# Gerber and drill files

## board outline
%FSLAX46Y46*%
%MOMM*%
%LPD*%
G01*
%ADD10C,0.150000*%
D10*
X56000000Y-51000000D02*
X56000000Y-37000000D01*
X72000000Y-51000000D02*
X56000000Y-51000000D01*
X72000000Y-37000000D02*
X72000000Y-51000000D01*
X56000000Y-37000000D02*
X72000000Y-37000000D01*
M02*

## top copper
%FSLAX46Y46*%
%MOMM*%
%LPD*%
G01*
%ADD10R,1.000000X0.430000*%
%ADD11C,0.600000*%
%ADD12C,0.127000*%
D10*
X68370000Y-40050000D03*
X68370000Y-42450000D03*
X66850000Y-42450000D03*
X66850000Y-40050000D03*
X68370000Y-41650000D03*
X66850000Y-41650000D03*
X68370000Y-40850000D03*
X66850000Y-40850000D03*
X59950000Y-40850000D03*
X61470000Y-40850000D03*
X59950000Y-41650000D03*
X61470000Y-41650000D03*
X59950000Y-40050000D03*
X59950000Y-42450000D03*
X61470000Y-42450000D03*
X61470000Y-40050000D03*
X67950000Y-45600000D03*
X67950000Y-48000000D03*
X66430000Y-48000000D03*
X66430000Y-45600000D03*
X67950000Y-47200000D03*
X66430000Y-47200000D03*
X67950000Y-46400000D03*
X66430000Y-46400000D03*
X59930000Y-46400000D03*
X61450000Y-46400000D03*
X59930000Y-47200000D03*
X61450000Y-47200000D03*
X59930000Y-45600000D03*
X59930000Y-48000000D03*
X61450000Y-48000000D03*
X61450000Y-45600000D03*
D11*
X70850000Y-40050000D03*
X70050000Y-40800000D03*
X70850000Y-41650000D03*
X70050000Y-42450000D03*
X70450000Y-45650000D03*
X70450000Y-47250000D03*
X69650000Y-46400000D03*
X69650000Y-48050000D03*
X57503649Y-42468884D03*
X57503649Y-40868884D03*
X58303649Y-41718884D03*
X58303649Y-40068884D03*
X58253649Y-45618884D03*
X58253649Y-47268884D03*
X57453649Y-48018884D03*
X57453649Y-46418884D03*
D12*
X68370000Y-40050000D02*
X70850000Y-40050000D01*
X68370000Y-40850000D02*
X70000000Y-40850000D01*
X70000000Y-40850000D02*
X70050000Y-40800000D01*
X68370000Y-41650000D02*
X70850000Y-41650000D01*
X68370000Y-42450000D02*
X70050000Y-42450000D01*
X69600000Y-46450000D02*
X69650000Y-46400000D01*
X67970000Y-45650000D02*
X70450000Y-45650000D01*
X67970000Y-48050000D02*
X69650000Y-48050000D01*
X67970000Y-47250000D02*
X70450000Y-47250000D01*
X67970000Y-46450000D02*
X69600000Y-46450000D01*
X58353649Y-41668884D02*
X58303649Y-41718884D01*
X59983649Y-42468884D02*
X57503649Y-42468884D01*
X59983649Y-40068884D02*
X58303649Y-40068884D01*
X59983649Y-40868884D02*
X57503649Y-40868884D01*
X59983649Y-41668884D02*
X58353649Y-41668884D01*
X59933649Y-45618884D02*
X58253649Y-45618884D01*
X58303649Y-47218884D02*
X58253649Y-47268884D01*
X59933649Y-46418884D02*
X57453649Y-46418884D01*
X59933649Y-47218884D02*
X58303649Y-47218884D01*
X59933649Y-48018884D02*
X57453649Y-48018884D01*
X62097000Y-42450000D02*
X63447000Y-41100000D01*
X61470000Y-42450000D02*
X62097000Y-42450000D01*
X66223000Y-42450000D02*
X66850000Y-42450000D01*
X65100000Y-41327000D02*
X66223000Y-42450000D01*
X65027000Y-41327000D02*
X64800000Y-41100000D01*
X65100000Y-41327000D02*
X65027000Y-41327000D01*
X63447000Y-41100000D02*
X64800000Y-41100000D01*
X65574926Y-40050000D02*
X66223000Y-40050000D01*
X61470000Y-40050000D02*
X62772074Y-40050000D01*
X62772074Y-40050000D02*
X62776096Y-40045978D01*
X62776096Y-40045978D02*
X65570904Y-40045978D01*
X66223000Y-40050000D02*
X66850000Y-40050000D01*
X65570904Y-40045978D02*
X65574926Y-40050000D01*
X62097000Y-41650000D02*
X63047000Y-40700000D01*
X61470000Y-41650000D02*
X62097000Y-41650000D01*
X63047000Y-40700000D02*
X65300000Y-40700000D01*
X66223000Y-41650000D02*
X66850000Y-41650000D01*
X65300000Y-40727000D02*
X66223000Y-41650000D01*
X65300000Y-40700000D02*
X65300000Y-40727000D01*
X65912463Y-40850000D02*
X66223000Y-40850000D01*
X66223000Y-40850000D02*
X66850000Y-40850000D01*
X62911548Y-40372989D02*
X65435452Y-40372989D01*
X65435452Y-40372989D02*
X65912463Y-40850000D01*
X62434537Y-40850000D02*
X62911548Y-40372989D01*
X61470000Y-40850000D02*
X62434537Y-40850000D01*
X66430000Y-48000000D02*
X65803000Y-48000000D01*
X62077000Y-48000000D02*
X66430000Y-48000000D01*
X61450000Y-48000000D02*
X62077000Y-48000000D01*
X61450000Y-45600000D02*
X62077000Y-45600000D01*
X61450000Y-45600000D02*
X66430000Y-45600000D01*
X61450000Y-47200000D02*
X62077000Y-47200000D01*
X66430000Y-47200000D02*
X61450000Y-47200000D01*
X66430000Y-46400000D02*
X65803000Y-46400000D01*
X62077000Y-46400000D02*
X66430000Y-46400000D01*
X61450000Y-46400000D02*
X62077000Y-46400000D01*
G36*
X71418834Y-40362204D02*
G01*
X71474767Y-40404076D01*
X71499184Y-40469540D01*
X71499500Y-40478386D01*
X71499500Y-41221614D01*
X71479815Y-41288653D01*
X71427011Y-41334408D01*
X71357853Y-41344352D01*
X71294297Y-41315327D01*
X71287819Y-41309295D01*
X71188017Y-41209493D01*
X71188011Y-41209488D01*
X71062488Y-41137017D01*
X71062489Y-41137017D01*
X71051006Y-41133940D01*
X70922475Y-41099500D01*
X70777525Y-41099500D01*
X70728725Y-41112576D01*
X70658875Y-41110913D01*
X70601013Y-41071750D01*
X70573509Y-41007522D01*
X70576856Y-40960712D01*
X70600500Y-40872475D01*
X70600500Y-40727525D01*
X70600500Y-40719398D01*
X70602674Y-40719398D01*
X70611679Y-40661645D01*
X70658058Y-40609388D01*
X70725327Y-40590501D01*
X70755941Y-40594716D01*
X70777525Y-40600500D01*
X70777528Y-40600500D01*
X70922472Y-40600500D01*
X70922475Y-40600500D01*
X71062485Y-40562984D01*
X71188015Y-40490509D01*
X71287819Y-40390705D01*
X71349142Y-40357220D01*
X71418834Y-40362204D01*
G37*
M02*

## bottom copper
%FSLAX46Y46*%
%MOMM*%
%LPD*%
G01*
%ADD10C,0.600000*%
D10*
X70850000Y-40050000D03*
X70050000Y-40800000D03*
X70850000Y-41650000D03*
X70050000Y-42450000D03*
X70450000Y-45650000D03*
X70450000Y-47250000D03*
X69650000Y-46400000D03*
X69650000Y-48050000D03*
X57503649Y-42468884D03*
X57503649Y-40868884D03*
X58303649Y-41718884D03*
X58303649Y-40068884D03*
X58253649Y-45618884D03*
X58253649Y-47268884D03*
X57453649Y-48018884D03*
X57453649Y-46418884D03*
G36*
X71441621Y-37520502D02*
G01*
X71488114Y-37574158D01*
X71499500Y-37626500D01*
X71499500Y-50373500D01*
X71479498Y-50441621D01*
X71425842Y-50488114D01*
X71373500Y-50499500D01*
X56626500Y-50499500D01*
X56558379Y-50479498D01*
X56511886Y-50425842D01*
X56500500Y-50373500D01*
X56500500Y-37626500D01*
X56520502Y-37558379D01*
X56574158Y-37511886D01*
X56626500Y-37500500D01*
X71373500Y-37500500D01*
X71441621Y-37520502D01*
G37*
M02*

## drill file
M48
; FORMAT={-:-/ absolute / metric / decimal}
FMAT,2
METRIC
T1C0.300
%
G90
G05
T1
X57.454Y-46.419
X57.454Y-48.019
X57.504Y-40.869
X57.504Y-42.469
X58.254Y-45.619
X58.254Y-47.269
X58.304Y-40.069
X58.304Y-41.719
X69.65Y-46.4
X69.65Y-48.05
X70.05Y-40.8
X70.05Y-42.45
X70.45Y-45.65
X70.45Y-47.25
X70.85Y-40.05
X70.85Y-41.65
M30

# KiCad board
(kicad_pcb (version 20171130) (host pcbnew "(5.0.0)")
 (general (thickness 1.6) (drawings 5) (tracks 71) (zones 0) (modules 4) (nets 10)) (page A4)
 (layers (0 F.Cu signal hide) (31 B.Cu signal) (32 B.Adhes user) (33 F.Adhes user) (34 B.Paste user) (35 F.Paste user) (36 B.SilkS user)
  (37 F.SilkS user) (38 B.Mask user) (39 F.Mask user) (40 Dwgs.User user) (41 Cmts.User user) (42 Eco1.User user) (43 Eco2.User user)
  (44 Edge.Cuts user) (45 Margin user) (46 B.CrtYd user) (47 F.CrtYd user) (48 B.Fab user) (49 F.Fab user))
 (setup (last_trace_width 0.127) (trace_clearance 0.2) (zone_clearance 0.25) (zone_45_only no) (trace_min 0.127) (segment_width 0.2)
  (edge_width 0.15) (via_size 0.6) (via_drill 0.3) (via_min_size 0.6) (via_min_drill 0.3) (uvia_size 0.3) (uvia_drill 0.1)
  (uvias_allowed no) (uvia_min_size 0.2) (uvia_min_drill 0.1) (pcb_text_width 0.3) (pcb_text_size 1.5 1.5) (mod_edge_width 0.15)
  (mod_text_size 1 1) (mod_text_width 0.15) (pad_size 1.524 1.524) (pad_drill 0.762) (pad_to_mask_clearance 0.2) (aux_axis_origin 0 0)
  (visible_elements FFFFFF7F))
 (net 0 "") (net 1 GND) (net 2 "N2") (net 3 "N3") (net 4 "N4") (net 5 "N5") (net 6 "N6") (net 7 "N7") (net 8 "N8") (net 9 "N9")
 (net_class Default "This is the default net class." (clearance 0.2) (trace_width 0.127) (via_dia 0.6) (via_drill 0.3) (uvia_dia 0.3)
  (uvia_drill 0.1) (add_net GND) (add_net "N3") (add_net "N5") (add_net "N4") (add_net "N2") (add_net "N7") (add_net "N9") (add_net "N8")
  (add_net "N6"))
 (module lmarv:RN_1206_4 (layer F.Cu) (at 67.61 41.25)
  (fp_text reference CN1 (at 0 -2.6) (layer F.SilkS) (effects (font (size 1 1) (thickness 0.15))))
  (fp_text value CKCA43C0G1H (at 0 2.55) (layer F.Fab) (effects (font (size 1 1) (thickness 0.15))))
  (pad 8 smd rect (at 0.76 -1.2 180) (size 1 0.43) (layers F.Cu F.Paste F.Mask) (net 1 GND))
  (pad 5 smd rect (at 0.76 1.2 180) (size 1 0.43) (layers F.Cu F.Paste F.Mask) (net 1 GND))
  (pad 4 smd rect (at -0.76 1.2 180) (size 1 0.43) (layers F.Cu F.Paste F.Mask) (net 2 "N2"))
  (pad 1 smd rect (at -0.76 -1.2 180) (size 1 0.43) (layers F.Cu F.Paste F.Mask) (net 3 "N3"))
  (pad 6 smd rect (at 0.76 0.4 180) (size 1 0.43) (layers F.Cu F.Paste F.Mask) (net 1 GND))
  (pad 3 smd rect (at -0.76 0.4 180) (size 1 0.43) (layers F.Cu F.Paste F.Mask) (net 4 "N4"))
  (pad 7 smd rect (at 0.76 -0.4 180) (size 1 0.43) (layers F.Cu F.Paste F.Mask) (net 1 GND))
  (pad 2 smd rect (at -0.76 -0.4 180) (size 1 0.43) (layers F.Cu F.Paste F.Mask) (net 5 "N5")))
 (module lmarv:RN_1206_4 (layer F.Cu) (at 60.71 41.25)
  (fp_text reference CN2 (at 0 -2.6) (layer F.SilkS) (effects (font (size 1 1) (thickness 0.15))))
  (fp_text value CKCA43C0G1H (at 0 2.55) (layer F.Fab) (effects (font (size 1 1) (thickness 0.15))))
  (pad 2 smd rect (at -0.76 -0.4 180) (size 1 0.43) (layers F.Cu F.Paste F.Mask) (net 1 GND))
  (pad 7 smd rect (at 0.76 -0.4 180) (size 1 0.43) (layers F.Cu F.Paste F.Mask) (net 5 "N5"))
  (pad 3 smd rect (at -0.76 0.4 180) (size 1 0.43) (layers F.Cu F.Paste F.Mask) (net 1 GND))
  (pad 6 smd rect (at 0.76 0.4 180) (size 1 0.43) (layers F.Cu F.Paste F.Mask) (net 4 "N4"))
  (pad 1 smd rect (at -0.76 -1.2 180) (size 1 0.43) (layers F.Cu F.Paste F.Mask) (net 1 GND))
  (pad 4 smd rect (at -0.76 1.2 180) (size 1 0.43) (layers F.Cu F.Paste F.Mask) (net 1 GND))
  (pad 5 smd rect (at 0.76 1.2 180) (size 1 0.43) (layers F.Cu F.Paste F.Mask) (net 2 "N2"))
  (pad 8 smd rect (at 0.76 -1.2 180) (size 1 0.43) (layers F.Cu F.Paste F.Mask) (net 3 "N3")))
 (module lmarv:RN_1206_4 (layer F.Cu) (at 67.19 46.8)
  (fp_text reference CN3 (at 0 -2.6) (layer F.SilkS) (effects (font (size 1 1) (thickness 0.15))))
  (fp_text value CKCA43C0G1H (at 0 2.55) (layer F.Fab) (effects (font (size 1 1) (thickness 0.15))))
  (pad 8 smd rect (at 0.76 -1.2 180) (size 1 0.43) (layers F.Cu F.Paste F.Mask) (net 1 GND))
  (pad 5 smd rect (at 0.76 1.2 180) (size 1 0.43) (layers F.Cu F.Paste F.Mask) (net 1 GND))
  (pad 4 smd rect (at -0.76 1.2 180) (size 1 0.43) (layers F.Cu F.Paste F.Mask) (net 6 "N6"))
  (pad 1 smd rect (at -0.76 -1.2 180) (size 1 0.43) (layers F.Cu F.Paste F.Mask) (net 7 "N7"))
  (pad 6 smd rect (at 0.76 0.4 180) (size 1 0.43) (layers F.Cu F.Paste F.Mask) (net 1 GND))
  (pad 3 smd rect (at -0.76 0.4 180) (size 1 0.43) (layers F.Cu F.Paste F.Mask) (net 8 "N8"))
  (pad 7 smd rect (at 0.76 -0.4 180) (size 1 0.43) (layers F.Cu F.Paste F.Mask) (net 1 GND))
  (pad 2 smd rect (at -0.76 -0.4 180) (size 1 0.43) (layers F.Cu F.Paste F.Mask) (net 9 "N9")))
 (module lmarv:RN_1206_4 (layer F.Cu) (at 60.69 46.8)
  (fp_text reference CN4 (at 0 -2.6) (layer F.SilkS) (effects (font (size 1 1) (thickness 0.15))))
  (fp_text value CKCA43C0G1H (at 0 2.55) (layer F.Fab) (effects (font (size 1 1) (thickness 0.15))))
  (pad 2 smd rect (at -0.76 -0.4 180) (size 1 0.43) (layers F.Cu F.Paste F.Mask) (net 1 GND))
  (pad 7 smd rect (at 0.76 -0.4 180) (size 1 0.43) (layers F.Cu F.Paste F.Mask) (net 9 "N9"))
  (pad 3 smd rect (at -0.76 0.4 180) (size 1 0.43) (layers F.Cu F.Paste F.Mask) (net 1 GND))
  (pad 6 smd rect (at 0.76 0.4 180) (size 1 0.43) (layers F.Cu F.Paste F.Mask) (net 8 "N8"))
  (pad 1 smd rect (at -0.76 -1.2 180) (size 1 0.43) (layers F.Cu F.Paste F.Mask) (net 1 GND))
  (pad 4 smd rect (at -0.76 1.2 180) (size 1 0.43) (layers F.Cu F.Paste F.Mask) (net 1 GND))
  (pad 5 smd rect (at 0.76 1.2 180) (size 1 0.43) (layers F.Cu F.Paste F.Mask) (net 6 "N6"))
  (pad 8 smd rect (at 0.76 -1.2 180) (size 1 0.43) (layers F.Cu F.Paste F.Mask) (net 7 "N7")))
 (gr_line (start 56 51) (end 56 37) (layer Edge.Cuts) (width 0.15))
 (gr_line (start 72 51) (end 56 51) (layer Edge.Cuts) (width 0.15))
 (gr_line (start 72 37) (end 72 51) (layer Edge.Cuts) (width 0.15))
 (gr_line (start 56 37) (end 72 37) (layer Edge.Cuts) (width 0.15))
 (via (at 70.85 40.05) (size 0.6) (drill 0.3) (layers F.Cu B.Cu) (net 1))
 (segment (start 68.37 40.05) (end 70.85 40.05) (width 0.127) (layer F.Cu) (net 1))
 (via (at 70.05 40.8) (size 0.6) (drill 0.3) (layers F.Cu B.Cu) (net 1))
 (segment (start 68.37 40.85) (end 70 40.85) (width 0.127) (layer F.Cu) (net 1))
 (segment (start 70 40.85) (end 70.05 40.8) (width 0.127) (layer F.Cu) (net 1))
 (via (at 70.85 41.65) (size 0.6) (drill 0.3) (layers F.Cu B.Cu) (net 1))
 (segment (start 68.37 41.65) (end 70.85 41.65) (width 0.127) (layer F.Cu) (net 1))
 (via (at 70.05 42.45) (size 0.6) (drill 0.3) (layers F.Cu B.Cu) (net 1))
 (segment (start 68.37 42.45) (end 70.05 42.45) (width 0.127) (layer F.Cu) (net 1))
 (via (at 70.45 45.65) (size 0.6) (drill 0.3) (layers F.Cu B.Cu) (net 1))
 (via (at 70.45 47.25) (size 0.6) (drill 0.3) (layers F.Cu B.Cu) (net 1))
 (via (at 69.65 46.4) (size 0.6) (drill 0.3) (layers F.Cu B.Cu) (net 1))
 (segment (start 69.6 46.45) (end 69.65 46.4) (width 0.127) (layer F.Cu) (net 1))
 (segment (start 67.97 45.65) (end 70.45 45.65) (width 0.127) (layer F.Cu) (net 1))
 (segment (start 67.97 48.05) (end 69.65 48.05) (width 0.127) (layer F.Cu) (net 1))
 (segment (start 67.97 47.25) (end 70.45 47.25) (width 0.127) (layer F.Cu) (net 1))
 (segment (start 67.97 46.45) (end 69.6 46.45) (width 0.127) (layer F.Cu) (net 1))
 (via (at 69.65 48.05) (size 0.6) (drill 0.3) (layers F.Cu B.Cu) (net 1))
 (via (at 57.503649 42.468884) (size 0.6) (drill 0.3) (layers F.Cu B.Cu) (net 1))
 (via (at 57.503649 40.868884) (size 0.6) (drill 0.3) (layers F.Cu B.Cu) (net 1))
 (via (at 58.303649 41.718884) (size 0.6) (drill 0.3) (layers F.Cu B.Cu) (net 1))
 (segment (start 58.353649 41.668884) (end 58.303649 41.718884) (width 0.127) (layer F.Cu) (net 1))
 (segment (start 59.983649 42.468884) (end 57.503649 42.468884) (width 0.127) (layer F.Cu) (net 1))
 (segment (start 59.983649 40.068884) (end 58.303649 40.068884) (width 0.127) (layer F.Cu) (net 1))
 (segment (start 59.983649 40.868884) (end 57.503649 40.868884) (width 0.127) (layer F.Cu) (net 1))
 (segment (start 59.983649 41.668884) (end 58.353649 41.668884) (width 0.127) (layer F.Cu) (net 1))
 (via (at 58.303649 40.068884) (size 0.6) (drill 0.3) (layers F.Cu B.Cu) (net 1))
 (segment (start 59.933649 45.618884) (end 58.253649 45.618884) (width 0.127) (layer F.Cu) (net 1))
 (segment (start 58.303649 47.218884) (end 58.253649 47.268884) (width 0.127) (layer F.Cu) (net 1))
 (segment (start 59.933649 46.418884) (end 57.453649 46.418884) (width 0.127) (layer F.Cu) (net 1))
 (segment (start 59.933649 47.218884) (end 58.303649 47.218884) (width 0.127) (layer F.Cu) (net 1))
 (segment (start 59.933649 48.018884) (end 57.453649 48.018884) (width 0.127) (layer F.Cu) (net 1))
 (via (at 58.253649 45.618884) (size 0.6) (drill 0.3) (layers F.Cu B.Cu) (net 1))
 (via (at 58.253649 47.268884) (size 0.6) (drill 0.3) (layers F.Cu B.Cu) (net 1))
 (via (at 57.453649 48.018884) (size 0.6) (drill 0.3) (layers F.Cu B.Cu) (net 1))
 (via (at 57.453649 46.418884) (size 0.6) (drill 0.3) (layers F.Cu B.Cu) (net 1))
 (segment (start 62.097 42.45) (end 63.447 41.1) (width 0.127) (layer F.Cu) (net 2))
 (segment (start 61.47 42.45) (end 62.097 42.45) (width 0.127) (layer F.Cu) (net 2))
 (segment (start 66.223 42.45) (end 66.85 42.45) (width 0.127) (layer F.Cu) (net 2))
 (segment (start 65.1 41.327) (end 66.223 42.45) (width 0.127) (layer F.Cu) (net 2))
 (segment (start 65.027 41.327) (end 64.8 41.1) (width 0.127) (layer F.Cu) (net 2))
 (segment (start 65.1 41.327) (end 65.027 41.327) (width 0.127) (layer F.Cu) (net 2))
 (segment (start 63.447 41.1) (end 64.8 41.1) (width 0.127) (layer F.Cu) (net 2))
 (segment (start 65.574926 40.05) (end 66.223 40.05) (width 0.127) (layer F.Cu) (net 3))
 (segment (start 61.47 40.05) (end 62.772074 40.05) (width 0.127) (layer F.Cu) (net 3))
 (segment (start 62.772074 40.05) (end 62.776096 40.045978) (width 0.127) (layer F.Cu) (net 3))
 (segment (start 62.776096 40.045978) (end 65.570904 40.045978) (width 0.127) (layer F.Cu) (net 3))
 (segment (start 66.223 40.05) (end 66.85 40.05) (width 0.127) (layer F.Cu) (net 3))
 (segment (start 65.570904 40.045978) (end 65.574926 40.05) (width 0.127) (layer F.Cu) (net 3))
 (segment (start 62.097 41.65) (end 63.047 40.7) (width 0.127) (layer F.Cu) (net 4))
 (segment (start 61.47 41.65) (end 62.097 41.65) (width 0.127) (layer F.Cu) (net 4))
 (segment (start 63.047 40.7) (end 65.3 40.7) (width 0.127) (layer F.Cu) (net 4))
 (segment (start 66.223 41.65) (end 66.85 41.65) (width 0.127) (layer F.Cu) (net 4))
 (segment (start 65.3 40.727) (end 66.223 41.65) (width 0.127) (layer F.Cu) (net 4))
 (segment (start 65.3 40.7) (end 65.3 40.727) (width 0.127) (layer F.Cu) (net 4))
 (segment (start 65.912463 40.85) (end 66.223 40.85) (width 0.127) (layer F.Cu) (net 5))
 (segment (start 66.223 40.85) (end 66.85 40.85) (width 0.127) (layer F.Cu) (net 5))
 (segment (start 62.911548 40.372989) (end 65.435452 40.372989) (width 0.127) (layer F.Cu) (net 5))
 (segment (start 65.435452 40.372989) (end 65.912463 40.85) (width 0.127) (layer F.Cu) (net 5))
 (segment (start 62.434537 40.85) (end 62.911548 40.372989) (width 0.127) (layer F.Cu) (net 5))
 (segment (start 61.47 40.85) (end 62.434537 40.85) (width 0.127) (layer F.Cu) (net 5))
 (segment (start 66.43 48) (end 65.803 48) (width 0.127) (layer F.Cu) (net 6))
 (segment (start 62.077 48) (end 66.43 48) (width 0.127) (layer F.Cu) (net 6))
 (segment (start 61.45 48) (end 62.077 48) (width 0.127) (layer F.Cu) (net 6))
 (segment (start 61.45 45.6) (end 62.077 45.6) (width 0.127) (layer F.Cu) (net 7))
 (segment (start 61.45 45.6) (end 66.43 45.6) (width 0.127) (layer F.Cu) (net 7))
 (segment (start 61.45 47.2) (end 62.077 47.2) (width 0.127) (layer F.Cu) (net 8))
 (segment (start 66.43 47.2) (end 61.45 47.2) (width 0.127) (layer F.Cu) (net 8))
 (segment (start 66.43 46.4) (end 65.803 46.4) (width 0.127) (layer F.Cu) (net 9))
 (segment (start 62.077 46.4) (end 66.43 46.4) (width 0.127) (layer F.Cu) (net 9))
 (segment (start 61.45 46.4) (end 62.077 46.4) (width 0.127) (layer F.Cu) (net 9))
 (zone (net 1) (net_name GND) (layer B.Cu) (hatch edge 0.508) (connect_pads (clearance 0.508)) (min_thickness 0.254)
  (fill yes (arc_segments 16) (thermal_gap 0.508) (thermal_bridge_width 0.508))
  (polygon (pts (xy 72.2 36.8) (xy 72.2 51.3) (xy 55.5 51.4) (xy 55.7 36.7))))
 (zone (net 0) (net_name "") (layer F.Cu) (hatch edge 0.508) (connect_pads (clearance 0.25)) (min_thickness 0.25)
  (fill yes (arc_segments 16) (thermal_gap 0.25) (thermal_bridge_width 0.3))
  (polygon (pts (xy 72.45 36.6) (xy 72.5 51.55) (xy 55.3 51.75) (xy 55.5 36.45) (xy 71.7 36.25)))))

